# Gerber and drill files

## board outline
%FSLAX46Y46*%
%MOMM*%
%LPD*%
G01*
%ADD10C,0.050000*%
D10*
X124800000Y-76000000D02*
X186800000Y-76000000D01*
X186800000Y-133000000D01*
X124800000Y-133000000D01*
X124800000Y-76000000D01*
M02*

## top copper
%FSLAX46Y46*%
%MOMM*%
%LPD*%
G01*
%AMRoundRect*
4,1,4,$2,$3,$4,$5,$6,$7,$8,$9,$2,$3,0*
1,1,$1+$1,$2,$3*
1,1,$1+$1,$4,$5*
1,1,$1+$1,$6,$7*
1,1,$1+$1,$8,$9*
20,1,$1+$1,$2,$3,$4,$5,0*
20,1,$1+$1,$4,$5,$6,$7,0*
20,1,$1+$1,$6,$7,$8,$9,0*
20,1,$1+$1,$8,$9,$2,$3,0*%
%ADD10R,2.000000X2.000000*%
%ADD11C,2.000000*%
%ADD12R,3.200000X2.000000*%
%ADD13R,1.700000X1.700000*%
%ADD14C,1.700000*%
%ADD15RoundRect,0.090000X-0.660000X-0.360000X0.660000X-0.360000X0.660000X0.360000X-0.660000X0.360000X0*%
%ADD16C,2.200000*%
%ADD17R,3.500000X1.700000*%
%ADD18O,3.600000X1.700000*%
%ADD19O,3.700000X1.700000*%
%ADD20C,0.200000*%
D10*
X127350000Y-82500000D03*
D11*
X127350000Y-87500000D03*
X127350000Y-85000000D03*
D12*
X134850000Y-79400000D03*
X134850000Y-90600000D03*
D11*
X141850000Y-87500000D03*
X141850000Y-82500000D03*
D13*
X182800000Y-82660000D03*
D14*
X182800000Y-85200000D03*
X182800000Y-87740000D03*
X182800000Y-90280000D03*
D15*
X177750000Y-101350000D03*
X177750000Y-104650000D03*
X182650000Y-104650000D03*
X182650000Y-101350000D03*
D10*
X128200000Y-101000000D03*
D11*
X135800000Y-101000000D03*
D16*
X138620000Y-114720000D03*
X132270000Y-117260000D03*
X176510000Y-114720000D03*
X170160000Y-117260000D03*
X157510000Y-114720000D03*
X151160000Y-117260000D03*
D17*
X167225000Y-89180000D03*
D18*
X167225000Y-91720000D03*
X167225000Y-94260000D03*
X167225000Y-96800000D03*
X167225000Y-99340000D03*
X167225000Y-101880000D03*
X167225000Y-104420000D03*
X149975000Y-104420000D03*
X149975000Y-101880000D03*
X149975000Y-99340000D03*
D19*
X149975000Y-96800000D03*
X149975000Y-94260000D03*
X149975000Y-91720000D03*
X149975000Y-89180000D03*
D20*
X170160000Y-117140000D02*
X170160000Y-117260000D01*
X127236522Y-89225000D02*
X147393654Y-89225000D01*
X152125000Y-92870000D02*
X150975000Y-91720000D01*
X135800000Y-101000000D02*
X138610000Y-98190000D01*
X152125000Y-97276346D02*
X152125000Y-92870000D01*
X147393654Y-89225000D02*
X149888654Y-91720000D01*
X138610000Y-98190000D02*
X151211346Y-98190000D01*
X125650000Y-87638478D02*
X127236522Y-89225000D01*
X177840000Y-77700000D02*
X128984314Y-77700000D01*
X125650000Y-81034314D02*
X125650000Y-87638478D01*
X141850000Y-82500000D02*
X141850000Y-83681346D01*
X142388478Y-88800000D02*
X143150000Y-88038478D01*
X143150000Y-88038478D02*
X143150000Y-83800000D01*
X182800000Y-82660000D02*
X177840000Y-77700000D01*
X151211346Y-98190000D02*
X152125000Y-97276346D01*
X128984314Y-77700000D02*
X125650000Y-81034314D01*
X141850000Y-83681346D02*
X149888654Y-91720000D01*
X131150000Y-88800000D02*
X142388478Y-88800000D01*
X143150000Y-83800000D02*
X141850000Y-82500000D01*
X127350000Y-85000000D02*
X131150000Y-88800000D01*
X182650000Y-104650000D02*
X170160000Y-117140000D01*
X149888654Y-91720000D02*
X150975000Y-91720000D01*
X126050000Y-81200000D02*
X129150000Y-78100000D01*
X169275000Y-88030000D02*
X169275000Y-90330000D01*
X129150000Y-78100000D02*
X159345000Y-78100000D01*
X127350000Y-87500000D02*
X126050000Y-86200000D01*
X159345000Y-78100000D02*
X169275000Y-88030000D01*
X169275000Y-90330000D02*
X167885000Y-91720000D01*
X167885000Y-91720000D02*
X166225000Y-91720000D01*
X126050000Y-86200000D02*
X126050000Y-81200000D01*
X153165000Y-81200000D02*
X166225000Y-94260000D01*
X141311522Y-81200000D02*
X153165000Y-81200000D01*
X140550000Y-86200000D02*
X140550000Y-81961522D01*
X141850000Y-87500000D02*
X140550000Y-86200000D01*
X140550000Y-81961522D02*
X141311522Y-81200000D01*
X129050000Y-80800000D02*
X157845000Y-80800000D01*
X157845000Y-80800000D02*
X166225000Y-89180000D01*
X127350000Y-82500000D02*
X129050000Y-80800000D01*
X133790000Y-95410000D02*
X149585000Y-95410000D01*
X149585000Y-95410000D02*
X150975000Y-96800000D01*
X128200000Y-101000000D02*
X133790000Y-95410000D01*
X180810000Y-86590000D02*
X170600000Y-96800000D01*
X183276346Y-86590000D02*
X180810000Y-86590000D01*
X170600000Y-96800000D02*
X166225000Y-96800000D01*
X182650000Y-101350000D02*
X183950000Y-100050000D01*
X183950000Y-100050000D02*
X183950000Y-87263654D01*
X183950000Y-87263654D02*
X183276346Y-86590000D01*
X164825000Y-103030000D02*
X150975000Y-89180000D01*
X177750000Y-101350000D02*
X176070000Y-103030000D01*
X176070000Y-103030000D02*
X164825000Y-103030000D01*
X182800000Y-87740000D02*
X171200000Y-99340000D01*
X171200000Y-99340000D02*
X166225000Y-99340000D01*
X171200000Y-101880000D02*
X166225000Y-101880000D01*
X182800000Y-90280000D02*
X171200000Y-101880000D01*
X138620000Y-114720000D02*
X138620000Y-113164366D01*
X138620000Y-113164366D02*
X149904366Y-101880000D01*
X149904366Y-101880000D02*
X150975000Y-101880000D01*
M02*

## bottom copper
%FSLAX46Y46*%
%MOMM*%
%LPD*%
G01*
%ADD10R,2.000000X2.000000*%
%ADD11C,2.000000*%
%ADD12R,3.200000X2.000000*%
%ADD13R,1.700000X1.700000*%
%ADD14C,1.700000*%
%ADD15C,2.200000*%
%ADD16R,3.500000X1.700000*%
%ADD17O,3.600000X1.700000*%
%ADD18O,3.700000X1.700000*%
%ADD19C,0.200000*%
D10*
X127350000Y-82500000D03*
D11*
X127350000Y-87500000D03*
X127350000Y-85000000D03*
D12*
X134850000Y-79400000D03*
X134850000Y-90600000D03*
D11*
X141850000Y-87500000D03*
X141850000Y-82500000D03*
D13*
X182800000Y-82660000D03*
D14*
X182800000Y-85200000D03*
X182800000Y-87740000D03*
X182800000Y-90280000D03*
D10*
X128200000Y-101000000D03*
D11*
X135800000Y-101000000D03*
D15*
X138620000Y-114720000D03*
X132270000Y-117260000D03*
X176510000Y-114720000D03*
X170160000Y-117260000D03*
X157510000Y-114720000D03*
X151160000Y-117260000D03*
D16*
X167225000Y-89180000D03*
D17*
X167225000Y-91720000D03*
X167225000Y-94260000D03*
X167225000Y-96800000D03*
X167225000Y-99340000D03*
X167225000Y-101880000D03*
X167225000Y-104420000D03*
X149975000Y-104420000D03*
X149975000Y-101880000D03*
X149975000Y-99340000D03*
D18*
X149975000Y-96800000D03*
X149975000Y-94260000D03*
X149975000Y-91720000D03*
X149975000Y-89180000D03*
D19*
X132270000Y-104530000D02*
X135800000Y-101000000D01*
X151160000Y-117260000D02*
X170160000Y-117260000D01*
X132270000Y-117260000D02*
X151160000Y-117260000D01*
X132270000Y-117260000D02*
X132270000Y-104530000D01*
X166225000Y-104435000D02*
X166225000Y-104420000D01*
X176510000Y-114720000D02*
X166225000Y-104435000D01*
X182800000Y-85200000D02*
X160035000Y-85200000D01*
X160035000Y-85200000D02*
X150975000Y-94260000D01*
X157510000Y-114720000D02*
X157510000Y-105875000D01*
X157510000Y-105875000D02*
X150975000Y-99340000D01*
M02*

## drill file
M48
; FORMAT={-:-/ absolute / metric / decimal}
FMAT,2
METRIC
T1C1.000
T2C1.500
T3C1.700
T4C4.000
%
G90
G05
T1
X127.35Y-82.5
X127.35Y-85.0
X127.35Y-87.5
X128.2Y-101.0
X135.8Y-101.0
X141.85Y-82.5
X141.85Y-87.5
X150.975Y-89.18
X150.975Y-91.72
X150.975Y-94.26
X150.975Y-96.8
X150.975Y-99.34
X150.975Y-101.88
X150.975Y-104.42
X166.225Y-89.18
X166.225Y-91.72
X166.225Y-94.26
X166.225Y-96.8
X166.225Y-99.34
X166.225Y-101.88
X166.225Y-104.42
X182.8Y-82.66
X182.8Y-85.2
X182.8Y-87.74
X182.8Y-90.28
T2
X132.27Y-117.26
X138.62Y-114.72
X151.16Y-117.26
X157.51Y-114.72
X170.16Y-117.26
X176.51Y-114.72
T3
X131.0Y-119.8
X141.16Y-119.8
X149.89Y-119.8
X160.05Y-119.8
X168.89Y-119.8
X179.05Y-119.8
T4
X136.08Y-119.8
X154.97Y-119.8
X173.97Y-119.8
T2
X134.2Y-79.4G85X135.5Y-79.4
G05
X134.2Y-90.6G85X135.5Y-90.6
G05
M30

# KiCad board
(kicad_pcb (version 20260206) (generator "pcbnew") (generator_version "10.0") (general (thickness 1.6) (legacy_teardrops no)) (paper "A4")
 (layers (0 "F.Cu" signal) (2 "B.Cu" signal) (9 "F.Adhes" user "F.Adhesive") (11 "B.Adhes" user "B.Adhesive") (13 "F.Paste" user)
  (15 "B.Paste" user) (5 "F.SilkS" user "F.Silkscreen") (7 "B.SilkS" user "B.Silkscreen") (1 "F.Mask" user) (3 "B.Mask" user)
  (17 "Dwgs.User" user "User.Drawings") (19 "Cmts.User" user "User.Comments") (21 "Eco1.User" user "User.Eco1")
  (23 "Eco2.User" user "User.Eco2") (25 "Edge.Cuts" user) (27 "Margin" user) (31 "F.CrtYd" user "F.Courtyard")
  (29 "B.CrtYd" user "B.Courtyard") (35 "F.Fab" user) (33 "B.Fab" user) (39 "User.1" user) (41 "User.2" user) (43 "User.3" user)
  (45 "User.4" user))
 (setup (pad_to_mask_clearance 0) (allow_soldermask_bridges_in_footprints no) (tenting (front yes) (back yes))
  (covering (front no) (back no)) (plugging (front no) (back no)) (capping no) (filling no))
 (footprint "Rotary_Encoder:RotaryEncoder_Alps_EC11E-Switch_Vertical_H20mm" (layer "F.Cu") (at 127.35 82.5)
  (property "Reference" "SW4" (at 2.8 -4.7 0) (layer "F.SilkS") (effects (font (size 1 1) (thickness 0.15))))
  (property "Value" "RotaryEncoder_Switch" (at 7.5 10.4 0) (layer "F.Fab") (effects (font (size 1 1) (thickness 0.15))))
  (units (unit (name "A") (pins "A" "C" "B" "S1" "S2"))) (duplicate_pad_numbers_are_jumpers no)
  (pad "A" thru_hole rect (at 0 0) (size 2 2) (drill 1) (layers "*.Cu" "*.Mask") (remove_unused_layers no) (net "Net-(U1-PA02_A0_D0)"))
  (pad "B" thru_hole circle (at 0 5) (size 2 2) (drill 1) (layers "*.Cu" "*.Mask") (remove_unused_layers no) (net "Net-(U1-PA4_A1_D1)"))
  (pad "C" thru_hole circle (at 0 2.5) (size 2 2) (drill 1) (layers "*.Cu" "*.Mask") (remove_unused_layers no) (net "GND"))
  (pad "MP" thru_hole rect (at 7.5 -3.1) (size 3.2 2) (drill oval 2.8 1.5) (layers "*.Cu" "*.Mask") (remove_unused_layers no))
  (pad "MP" thru_hole rect (at 7.5 8.1) (size 3.2 2) (drill oval 2.8 1.5) (layers "*.Cu" "*.Mask") (remove_unused_layers no))
  (pad "S1" thru_hole circle (at 14.5 5) (size 2 2) (drill 1) (layers "*.Cu" "*.Mask") (remove_unused_layers no) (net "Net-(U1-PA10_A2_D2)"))
  (pad "S2" thru_hole circle (at 14.5 0) (size 2 2) (drill 1) (layers "*.Cu" "*.Mask") (remove_unused_layers no) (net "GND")))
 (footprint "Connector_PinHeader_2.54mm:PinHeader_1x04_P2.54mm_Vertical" (layer "F.Cu") (at 182.8 82.66)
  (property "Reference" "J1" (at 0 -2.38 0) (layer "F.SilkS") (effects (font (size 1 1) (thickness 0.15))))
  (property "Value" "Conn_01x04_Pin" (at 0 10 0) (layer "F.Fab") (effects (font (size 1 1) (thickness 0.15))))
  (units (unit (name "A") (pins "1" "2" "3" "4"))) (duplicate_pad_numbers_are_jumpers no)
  (pad "1" thru_hole rect (at 0 0) (size 1.7 1.7) (drill 1) (layers "*.Cu" "*.Mask") (remove_unused_layers no) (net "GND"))
  (pad "2" thru_hole circle (at 0 2.54) (size 1.7 1.7) (drill 1) (layers "*.Cu" "*.Mask") (remove_unused_layers no) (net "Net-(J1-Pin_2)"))
  (pad "3" thru_hole circle (at 0 5.08) (size 1.7 1.7) (drill 1) (layers "*.Cu" "*.Mask") (remove_unused_layers no) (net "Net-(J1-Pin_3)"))
  (pad "4" thru_hole circle (at 0 7.62) (size 1.7 1.7) (drill 1) (layers "*.Cu" "*.Mask") (remove_unused_layers no) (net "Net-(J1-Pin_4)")))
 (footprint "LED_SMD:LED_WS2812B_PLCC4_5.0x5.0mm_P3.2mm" (layer "F.Cu") (at 180.2 103)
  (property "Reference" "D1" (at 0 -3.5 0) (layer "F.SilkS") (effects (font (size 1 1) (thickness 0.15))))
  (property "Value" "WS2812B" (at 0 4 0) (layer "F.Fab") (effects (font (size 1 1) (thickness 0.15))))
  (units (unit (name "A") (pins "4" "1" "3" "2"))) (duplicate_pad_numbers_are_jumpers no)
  (pad "1" smd roundrect (at -2.45 -1.65) (size 1.5 0.9) (layers "F.Cu" "F.Mask" "F.Paste") (roundrect_rratio 0.1) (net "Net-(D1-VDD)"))
  (pad "2" smd roundrect (at -2.45 1.65) (size 1.5 0.9) (layers "F.Cu" "F.Mask" "F.Paste") (roundrect_rratio 0.1)
   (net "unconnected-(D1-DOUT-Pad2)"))
  (pad "3" smd roundrect (at 2.45 1.65) (size 1.5 0.9) (layers "F.Cu" "F.Mask" "F.Paste") (roundrect_rratio 0.1) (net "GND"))
  (pad "4" smd roundrect (at 2.45 -1.65) (size 1.5 0.9) (layers "F.Cu" "F.Mask" "F.Paste") (roundrect_rratio 0.1) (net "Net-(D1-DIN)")))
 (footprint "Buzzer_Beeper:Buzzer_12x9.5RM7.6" (layer "F.Cu") (at 128.2 101)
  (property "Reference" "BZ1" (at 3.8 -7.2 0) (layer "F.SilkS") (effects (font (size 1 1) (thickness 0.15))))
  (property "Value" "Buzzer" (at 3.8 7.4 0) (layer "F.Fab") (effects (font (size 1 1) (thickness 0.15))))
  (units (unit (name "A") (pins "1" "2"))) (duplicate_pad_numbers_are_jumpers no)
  (pad "1" thru_hole rect (at 0 0) (size 2 2) (drill 1) (layers "*.Cu" "*.Mask") (remove_unused_layers no) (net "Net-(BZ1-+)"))
  (pad "2" thru_hole circle (at 7.6 0) (size 2 2) (drill 1) (layers "*.Cu" "*.Mask") (remove_unused_layers no) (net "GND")))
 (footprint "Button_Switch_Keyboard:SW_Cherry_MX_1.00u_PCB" (layer "F.Cu") (at 138.62 114.72)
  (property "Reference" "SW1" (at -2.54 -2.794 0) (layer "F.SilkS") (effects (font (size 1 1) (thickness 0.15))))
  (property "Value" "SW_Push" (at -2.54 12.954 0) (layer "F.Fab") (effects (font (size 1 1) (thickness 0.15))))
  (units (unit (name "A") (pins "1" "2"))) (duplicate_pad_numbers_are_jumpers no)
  (pad "" np_thru_hole circle (at -7.62 5.08) (size 1.7 1.7) (drill 1.7) (layers "*.Cu" "*.Mask"))
  (pad "" np_thru_hole circle (at -2.54 5.08) (size 4 4) (drill 4) (layers "*.Cu" "*.Mask"))
  (pad "" np_thru_hole circle (at 2.54 5.08) (size 1.7 1.7) (drill 1.7) (layers "*.Cu" "*.Mask"))
  (pad "1" thru_hole circle (at 0 0) (size 2.2 2.2) (drill 1.5) (layers "*.Cu" "*.Mask") (remove_unused_layers no)
   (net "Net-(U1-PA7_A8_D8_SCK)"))
  (pad "2" thru_hole circle (at -6.35 2.54) (size 2.2 2.2) (drill 1.5) (layers "*.Cu" "*.Mask") (remove_unused_layers no) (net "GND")))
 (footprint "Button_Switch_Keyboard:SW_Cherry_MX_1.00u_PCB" (layer "F.Cu") (at 176.51 114.72)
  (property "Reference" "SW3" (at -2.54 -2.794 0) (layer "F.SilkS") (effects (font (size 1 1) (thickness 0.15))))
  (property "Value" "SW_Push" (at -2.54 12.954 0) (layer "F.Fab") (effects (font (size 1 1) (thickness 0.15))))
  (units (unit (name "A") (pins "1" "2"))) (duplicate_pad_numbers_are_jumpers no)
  (pad "" np_thru_hole circle (at -7.62 5.08) (size 1.7 1.7) (drill 1.7) (layers "*.Cu" "*.Mask"))
  (pad "" np_thru_hole circle (at -2.54 5.08) (size 4 4) (drill 4) (layers "*.Cu" "*.Mask"))
  (pad "" np_thru_hole circle (at 2.54 5.08) (size 1.7 1.7) (drill 1.7) (layers "*.Cu" "*.Mask"))
  (pad "1" thru_hole circle (at 0 0) (size 2.2 2.2) (drill 1.5) (layers "*.Cu" "*.Mask") (remove_unused_layers no)
   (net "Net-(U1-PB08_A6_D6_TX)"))
  (pad "2" thru_hole circle (at -6.35 2.54) (size 2.2 2.2) (drill 1.5) (layers "*.Cu" "*.Mask") (remove_unused_layers no) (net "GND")))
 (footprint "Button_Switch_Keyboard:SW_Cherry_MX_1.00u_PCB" (layer "F.Cu") (at 157.51 114.72)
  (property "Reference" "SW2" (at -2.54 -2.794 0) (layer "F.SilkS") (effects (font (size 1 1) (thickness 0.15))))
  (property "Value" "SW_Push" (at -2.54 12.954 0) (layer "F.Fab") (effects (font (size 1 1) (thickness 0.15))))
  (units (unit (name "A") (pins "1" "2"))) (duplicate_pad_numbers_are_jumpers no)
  (pad "" np_thru_hole circle (at -7.62 5.08) (size 1.7 1.7) (drill 1.7) (layers "*.Cu" "*.Mask"))
  (pad "" np_thru_hole circle (at -2.54 5.08) (size 4 4) (drill 4) (layers "*.Cu" "*.Mask"))
  (pad "" np_thru_hole circle (at 2.54 5.08) (size 1.7 1.7) (drill 1.7) (layers "*.Cu" "*.Mask"))
  (pad "1" thru_hole circle (at 0 0) (size 2.2 2.2) (drill 1.5) (layers "*.Cu" "*.Mask") (remove_unused_layers no)
   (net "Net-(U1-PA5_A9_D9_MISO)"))
  (pad "2" thru_hole circle (at -6.35 2.54) (size 2.2 2.2) (drill 1.5) (layers "*.Cu" "*.Mask") (remove_unused_layers no) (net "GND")))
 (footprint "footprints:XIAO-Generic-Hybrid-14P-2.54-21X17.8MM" (layer "B.Cu") (at 158.6 96.8 180)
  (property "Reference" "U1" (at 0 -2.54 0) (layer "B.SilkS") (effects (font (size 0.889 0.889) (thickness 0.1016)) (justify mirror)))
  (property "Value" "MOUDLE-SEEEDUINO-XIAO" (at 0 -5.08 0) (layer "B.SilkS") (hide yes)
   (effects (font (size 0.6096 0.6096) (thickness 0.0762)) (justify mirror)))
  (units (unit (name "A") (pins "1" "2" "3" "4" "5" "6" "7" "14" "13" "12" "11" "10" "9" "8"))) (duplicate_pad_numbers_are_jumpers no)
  (pad "1" thru_hole rect (at -7.625 7.62 180) (size 3.5 1.7) (drill 1 (offset -1 0)) (layers "*.Cu" "*.Mask") (remove_unused_layers no)
   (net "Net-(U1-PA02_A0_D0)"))
  (pad "2" thru_hole oval (at -7.625 5.08 180) (size 3.6 1.7) (drill 1 (offset -1 0)) (layers "*.Cu" "*.Mask") (remove_unused_layers no)
   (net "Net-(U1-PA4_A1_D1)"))
  (pad "3" thru_hole oval (at -7.625 2.54 180) (size 3.6 1.7) (drill 1 (offset -1 0)) (layers "*.Cu" "*.Mask") (remove_unused_layers no)
   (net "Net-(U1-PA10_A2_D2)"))
  (pad "4" thru_hole oval (at -7.625 0 180) (size 3.6 1.7) (drill 1 (offset -1 0)) (layers "*.Cu" "*.Mask") (remove_unused_layers no)
   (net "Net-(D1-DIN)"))
  (pad "5" thru_hole oval (at -7.625 -2.54 180) (size 3.6 1.7) (drill 1 (offset -1 0)) (layers "*.Cu" "*.Mask") (remove_unused_layers no)
   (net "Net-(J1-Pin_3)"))
  (pad "6" thru_hole oval (at -7.625 -5.08) (size 3.6 1.7) (drill 1 (offset 1 0)) (layers "*.Cu" "*.Mask") (remove_unused_layers no)
   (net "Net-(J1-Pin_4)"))
  (pad "7" thru_hole oval (at -7.625 -7.62 180) (size 3.6 1.7) (drill 1 (offset -1 0)) (layers "*.Cu" "*.Mask") (remove_unused_layers no)
   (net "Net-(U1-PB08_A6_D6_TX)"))
  (pad "8" thru_hole oval (at 7.625 -7.62 180) (size 3.6 1.7) (drill 1 (offset 1 0)) (layers "*.Cu" "*.Mask") (remove_unused_layers no)
   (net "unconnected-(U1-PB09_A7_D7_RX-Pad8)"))
  (pad "9" thru_hole oval (at 7.625 -5.08 180) (size 3.6 1.7) (drill 1 (offset 1 0)) (layers "*.Cu" "*.Mask") (remove_unused_layers no)
   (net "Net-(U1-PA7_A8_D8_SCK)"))
  (pad "10" thru_hole oval (at 7.625 -2.54 180) (size 3.6 1.7) (drill 1 (offset 1 0)) (layers "*.Cu" "*.Mask") (remove_unused_layers no)
   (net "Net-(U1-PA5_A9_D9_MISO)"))
  (pad "11" thru_hole oval (at 7.625 0 180) (size 3.7 1.7) (drill 1 (offset 1 0)) (layers "*.Cu" "*.Mask") (remove_unused_layers no)
   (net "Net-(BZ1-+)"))
  (pad "12" thru_hole oval (at 7.625 2.54 180) (size 3.7 1.7) (drill 1 (offset 1 0)) (layers "*.Cu" "*.Mask") (remove_unused_layers no)
   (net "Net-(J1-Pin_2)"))
  (pad "13" thru_hole oval (at 7.625 5.08 180) (size 3.7 1.7) (drill 1 (offset 1 0)) (layers "*.Cu" "*.Mask") (remove_unused_layers no)
   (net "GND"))
  (pad "14" thru_hole oval (at 7.625 7.62 180) (size 3.7 1.7) (drill 1 (offset 1 0)) (layers "*.Cu" "*.Mask") (remove_unused_layers no)
   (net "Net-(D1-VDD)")))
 (gr_rect (start 124.8 76) (end 186.8 133) (stroke (width 0.05) (type default)) (fill no) (layer "Edge.Cuts"))
 (segment (start 170.16 117.14) (end 170.16 117.26) (width 0.2) (layer "F.Cu") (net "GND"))
 (segment (start 127.236522 89.225) (end 147.393654 89.225) (width 0.2) (layer "F.Cu") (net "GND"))
 (segment (start 152.125 92.87) (end 150.975 91.72) (width 0.2) (layer "F.Cu") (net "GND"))
 (segment (start 135.8 101) (end 138.61 98.19) (width 0.2) (layer "F.Cu") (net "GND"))
 (segment (start 152.125 97.276346) (end 152.125 92.87) (width 0.2) (layer "F.Cu") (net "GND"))
 (segment (start 147.393654 89.225) (end 149.888654 91.72) (width 0.2) (layer "F.Cu") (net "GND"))
 (segment (start 138.61 98.19) (end 151.211346 98.19) (width 0.2) (layer "F.Cu") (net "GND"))
 (segment (start 125.65 87.638478) (end 127.236522 89.225) (width 0.2) (layer "F.Cu") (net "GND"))
 (segment (start 177.84 77.7) (end 128.984314 77.7) (width 0.2) (layer "F.Cu") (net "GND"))
 (segment (start 125.65 81.034314) (end 125.65 87.638478) (width 0.2) (layer "F.Cu") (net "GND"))
 (segment (start 141.85 82.5) (end 141.85 83.681346) (width 0.2) (layer "F.Cu") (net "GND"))
 (segment (start 142.388478 88.8) (end 143.15 88.038478) (width 0.2) (layer "F.Cu") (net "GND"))
 (segment (start 143.15 88.038478) (end 143.15 83.8) (width 0.2) (layer "F.Cu") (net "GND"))
 (segment (start 182.8 82.66) (end 177.84 77.7) (width 0.2) (layer "F.Cu") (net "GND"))
 (segment (start 151.211346 98.19) (end 152.125 97.276346) (width 0.2) (layer "F.Cu") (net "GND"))
 (segment (start 128.984314 77.7) (end 125.65 81.034314) (width 0.2) (layer "F.Cu") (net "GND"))
 (segment (start 141.85 83.681346) (end 149.888654 91.72) (width 0.2) (layer "F.Cu") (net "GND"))
 (segment (start 131.15 88.8) (end 142.388478 88.8) (width 0.2) (layer "F.Cu") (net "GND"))
 (segment (start 143.15 83.8) (end 141.85 82.5) (width 0.2) (layer "F.Cu") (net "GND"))
 (segment (start 127.35 85) (end 131.15 88.8) (width 0.2) (layer "F.Cu") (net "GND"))
 (segment (start 182.65 104.65) (end 170.16 117.14) (width 0.2) (layer "F.Cu") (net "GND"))
 (segment (start 149.888654 91.72) (end 150.975 91.72) (width 0.2) (layer "F.Cu") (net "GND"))
 (segment (start 132.27 104.53) (end 135.8 101) (width 0.2) (layer "B.Cu") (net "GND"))
 (segment (start 151.16 117.26) (end 170.16 117.26) (width 0.2) (layer "B.Cu") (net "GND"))
 (segment (start 132.27 117.26) (end 151.16 117.26) (width 0.2) (layer "B.Cu") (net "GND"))
 (segment (start 132.27 117.26) (end 132.27 104.53) (width 0.2) (layer "B.Cu") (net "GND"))
 (segment (start 166.225 104.435) (end 166.225 104.42) (width 0.2) (layer "B.Cu") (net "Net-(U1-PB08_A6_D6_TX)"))
 (segment (start 176.51 114.72) (end 166.225 104.435) (width 0.2) (layer "B.Cu") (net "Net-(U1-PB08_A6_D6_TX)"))
 (segment (start 126.05 81.2) (end 129.15 78.1) (width 0.2) (layer "F.Cu") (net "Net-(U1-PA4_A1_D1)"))
 (segment (start 169.275 88.03) (end 169.275 90.33) (width 0.2) (layer "F.Cu") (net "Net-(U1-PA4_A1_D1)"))
 (segment (start 129.15 78.1) (end 159.345 78.1) (width 0.2) (layer "F.Cu") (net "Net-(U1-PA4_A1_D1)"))
 (segment (start 127.35 87.5) (end 126.05 86.2) (width 0.2) (layer "F.Cu") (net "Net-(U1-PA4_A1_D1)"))
 (segment (start 159.345 78.1) (end 169.275 88.03) (width 0.2) (layer "F.Cu") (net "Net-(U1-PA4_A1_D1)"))
 (segment (start 169.275 90.33) (end 167.885 91.72) (width 0.2) (layer "F.Cu") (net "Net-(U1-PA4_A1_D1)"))
 (segment (start 167.885 91.72) (end 166.225 91.72) (width 0.2) (layer "F.Cu") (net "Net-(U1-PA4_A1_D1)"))
 (segment (start 126.05 86.2) (end 126.05 81.2) (width 0.2) (layer "F.Cu") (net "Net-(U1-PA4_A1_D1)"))
 (segment (start 153.165 81.2) (end 166.225 94.26) (width 0.2) (layer "F.Cu") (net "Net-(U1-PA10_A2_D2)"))
 (segment (start 141.311522 81.2) (end 153.165 81.2) (width 0.2) (layer "F.Cu") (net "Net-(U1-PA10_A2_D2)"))
 (segment (start 140.55 86.2) (end 140.55 81.961522) (width 0.2) (layer "F.Cu") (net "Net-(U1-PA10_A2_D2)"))
 (segment (start 141.85 87.5) (end 140.55 86.2) (width 0.2) (layer "F.Cu") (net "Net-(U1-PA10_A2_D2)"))
 (segment (start 140.55 81.961522) (end 141.311522 81.2) (width 0.2) (layer "F.Cu") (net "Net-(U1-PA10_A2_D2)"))
 (segment (start 129.05 80.8) (end 157.845 80.8) (width 0.2) (layer "F.Cu") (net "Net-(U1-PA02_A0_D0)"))
 (segment (start 157.845 80.8) (end 166.225 89.18) (width 0.2) (layer "F.Cu") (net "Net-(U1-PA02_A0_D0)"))
 (segment (start 127.35 82.5) (end 129.05 80.8) (width 0.2) (layer "F.Cu") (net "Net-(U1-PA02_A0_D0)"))
 (segment (start 133.79 95.41) (end 149.585 95.41) (width 0.2) (layer "F.Cu") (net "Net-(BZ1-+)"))
 (segment (start 149.585 95.41) (end 150.975 96.8) (width 0.2) (layer "F.Cu") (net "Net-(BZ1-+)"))
 (segment (start 128.2 101) (end 133.79 95.41) (width 0.2) (layer "F.Cu") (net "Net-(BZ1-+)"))
 (segment (start 180.81 86.59) (end 170.6 96.8) (width 0.2) (layer "F.Cu") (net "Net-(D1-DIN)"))
 (segment (start 183.276346 86.59) (end 180.81 86.59) (width 0.2) (layer "F.Cu") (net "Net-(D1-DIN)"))
 (segment (start 170.6 96.8) (end 166.225 96.8) (width 0.2) (layer "F.Cu") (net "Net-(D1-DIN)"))
 (segment (start 182.65 101.35) (end 183.95 100.05) (width 0.2) (layer "F.Cu") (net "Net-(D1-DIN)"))
 (segment (start 183.95 100.05) (end 183.95 87.263654) (width 0.2) (layer "F.Cu") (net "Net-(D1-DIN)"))
 (segment (start 183.95 87.263654) (end 183.276346 86.59) (width 0.2) (layer "F.Cu") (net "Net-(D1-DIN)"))
 (segment (start 164.825 103.03) (end 150.975 89.18) (width 0.2) (layer "F.Cu") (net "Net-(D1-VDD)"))
 (segment (start 177.75 101.35) (end 176.07 103.03) (width 0.2) (layer "F.Cu") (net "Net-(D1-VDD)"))
 (segment (start 176.07 103.03) (end 164.825 103.03) (width 0.2) (layer "F.Cu") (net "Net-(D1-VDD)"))
 (segment (start 182.8 85.2) (end 160.035 85.2) (width 0.2) (layer "B.Cu") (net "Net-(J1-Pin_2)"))
 (segment (start 160.035 85.2) (end 150.975 94.26) (width 0.2) (layer "B.Cu") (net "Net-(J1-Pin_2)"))
 (segment (start 182.8 87.74) (end 171.2 99.34) (width 0.2) (layer "F.Cu") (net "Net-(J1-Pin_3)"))
 (segment (start 171.2 99.34) (end 166.225 99.34) (width 0.2) (layer "F.Cu") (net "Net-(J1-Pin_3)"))
 (segment (start 171.2 101.88) (end 166.225 101.88) (width 0.2) (layer "F.Cu") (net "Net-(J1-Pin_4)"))
 (segment (start 182.8 90.28) (end 171.2 101.88) (width 0.2) (layer "F.Cu") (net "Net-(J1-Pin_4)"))
 (segment (start 138.62 114.72) (end 138.62 113.164366) (width 0.2) (layer "F.Cu") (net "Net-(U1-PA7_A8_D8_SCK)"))
 (segment (start 138.62 113.164366) (end 149.904366 101.88) (width 0.2) (layer "F.Cu") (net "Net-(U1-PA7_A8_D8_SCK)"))
 (segment (start 149.904366 101.88) (end 150.975 101.88) (width 0.2) (layer "F.Cu") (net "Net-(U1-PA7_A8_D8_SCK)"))
 (segment (start 157.51 114.72) (end 157.51 105.875) (width 0.2) (layer "B.Cu") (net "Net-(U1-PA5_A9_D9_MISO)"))
 (segment (start 157.51 105.875) (end 150.975 99.34) (width 0.2) (layer "B.Cu") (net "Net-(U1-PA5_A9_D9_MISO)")))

